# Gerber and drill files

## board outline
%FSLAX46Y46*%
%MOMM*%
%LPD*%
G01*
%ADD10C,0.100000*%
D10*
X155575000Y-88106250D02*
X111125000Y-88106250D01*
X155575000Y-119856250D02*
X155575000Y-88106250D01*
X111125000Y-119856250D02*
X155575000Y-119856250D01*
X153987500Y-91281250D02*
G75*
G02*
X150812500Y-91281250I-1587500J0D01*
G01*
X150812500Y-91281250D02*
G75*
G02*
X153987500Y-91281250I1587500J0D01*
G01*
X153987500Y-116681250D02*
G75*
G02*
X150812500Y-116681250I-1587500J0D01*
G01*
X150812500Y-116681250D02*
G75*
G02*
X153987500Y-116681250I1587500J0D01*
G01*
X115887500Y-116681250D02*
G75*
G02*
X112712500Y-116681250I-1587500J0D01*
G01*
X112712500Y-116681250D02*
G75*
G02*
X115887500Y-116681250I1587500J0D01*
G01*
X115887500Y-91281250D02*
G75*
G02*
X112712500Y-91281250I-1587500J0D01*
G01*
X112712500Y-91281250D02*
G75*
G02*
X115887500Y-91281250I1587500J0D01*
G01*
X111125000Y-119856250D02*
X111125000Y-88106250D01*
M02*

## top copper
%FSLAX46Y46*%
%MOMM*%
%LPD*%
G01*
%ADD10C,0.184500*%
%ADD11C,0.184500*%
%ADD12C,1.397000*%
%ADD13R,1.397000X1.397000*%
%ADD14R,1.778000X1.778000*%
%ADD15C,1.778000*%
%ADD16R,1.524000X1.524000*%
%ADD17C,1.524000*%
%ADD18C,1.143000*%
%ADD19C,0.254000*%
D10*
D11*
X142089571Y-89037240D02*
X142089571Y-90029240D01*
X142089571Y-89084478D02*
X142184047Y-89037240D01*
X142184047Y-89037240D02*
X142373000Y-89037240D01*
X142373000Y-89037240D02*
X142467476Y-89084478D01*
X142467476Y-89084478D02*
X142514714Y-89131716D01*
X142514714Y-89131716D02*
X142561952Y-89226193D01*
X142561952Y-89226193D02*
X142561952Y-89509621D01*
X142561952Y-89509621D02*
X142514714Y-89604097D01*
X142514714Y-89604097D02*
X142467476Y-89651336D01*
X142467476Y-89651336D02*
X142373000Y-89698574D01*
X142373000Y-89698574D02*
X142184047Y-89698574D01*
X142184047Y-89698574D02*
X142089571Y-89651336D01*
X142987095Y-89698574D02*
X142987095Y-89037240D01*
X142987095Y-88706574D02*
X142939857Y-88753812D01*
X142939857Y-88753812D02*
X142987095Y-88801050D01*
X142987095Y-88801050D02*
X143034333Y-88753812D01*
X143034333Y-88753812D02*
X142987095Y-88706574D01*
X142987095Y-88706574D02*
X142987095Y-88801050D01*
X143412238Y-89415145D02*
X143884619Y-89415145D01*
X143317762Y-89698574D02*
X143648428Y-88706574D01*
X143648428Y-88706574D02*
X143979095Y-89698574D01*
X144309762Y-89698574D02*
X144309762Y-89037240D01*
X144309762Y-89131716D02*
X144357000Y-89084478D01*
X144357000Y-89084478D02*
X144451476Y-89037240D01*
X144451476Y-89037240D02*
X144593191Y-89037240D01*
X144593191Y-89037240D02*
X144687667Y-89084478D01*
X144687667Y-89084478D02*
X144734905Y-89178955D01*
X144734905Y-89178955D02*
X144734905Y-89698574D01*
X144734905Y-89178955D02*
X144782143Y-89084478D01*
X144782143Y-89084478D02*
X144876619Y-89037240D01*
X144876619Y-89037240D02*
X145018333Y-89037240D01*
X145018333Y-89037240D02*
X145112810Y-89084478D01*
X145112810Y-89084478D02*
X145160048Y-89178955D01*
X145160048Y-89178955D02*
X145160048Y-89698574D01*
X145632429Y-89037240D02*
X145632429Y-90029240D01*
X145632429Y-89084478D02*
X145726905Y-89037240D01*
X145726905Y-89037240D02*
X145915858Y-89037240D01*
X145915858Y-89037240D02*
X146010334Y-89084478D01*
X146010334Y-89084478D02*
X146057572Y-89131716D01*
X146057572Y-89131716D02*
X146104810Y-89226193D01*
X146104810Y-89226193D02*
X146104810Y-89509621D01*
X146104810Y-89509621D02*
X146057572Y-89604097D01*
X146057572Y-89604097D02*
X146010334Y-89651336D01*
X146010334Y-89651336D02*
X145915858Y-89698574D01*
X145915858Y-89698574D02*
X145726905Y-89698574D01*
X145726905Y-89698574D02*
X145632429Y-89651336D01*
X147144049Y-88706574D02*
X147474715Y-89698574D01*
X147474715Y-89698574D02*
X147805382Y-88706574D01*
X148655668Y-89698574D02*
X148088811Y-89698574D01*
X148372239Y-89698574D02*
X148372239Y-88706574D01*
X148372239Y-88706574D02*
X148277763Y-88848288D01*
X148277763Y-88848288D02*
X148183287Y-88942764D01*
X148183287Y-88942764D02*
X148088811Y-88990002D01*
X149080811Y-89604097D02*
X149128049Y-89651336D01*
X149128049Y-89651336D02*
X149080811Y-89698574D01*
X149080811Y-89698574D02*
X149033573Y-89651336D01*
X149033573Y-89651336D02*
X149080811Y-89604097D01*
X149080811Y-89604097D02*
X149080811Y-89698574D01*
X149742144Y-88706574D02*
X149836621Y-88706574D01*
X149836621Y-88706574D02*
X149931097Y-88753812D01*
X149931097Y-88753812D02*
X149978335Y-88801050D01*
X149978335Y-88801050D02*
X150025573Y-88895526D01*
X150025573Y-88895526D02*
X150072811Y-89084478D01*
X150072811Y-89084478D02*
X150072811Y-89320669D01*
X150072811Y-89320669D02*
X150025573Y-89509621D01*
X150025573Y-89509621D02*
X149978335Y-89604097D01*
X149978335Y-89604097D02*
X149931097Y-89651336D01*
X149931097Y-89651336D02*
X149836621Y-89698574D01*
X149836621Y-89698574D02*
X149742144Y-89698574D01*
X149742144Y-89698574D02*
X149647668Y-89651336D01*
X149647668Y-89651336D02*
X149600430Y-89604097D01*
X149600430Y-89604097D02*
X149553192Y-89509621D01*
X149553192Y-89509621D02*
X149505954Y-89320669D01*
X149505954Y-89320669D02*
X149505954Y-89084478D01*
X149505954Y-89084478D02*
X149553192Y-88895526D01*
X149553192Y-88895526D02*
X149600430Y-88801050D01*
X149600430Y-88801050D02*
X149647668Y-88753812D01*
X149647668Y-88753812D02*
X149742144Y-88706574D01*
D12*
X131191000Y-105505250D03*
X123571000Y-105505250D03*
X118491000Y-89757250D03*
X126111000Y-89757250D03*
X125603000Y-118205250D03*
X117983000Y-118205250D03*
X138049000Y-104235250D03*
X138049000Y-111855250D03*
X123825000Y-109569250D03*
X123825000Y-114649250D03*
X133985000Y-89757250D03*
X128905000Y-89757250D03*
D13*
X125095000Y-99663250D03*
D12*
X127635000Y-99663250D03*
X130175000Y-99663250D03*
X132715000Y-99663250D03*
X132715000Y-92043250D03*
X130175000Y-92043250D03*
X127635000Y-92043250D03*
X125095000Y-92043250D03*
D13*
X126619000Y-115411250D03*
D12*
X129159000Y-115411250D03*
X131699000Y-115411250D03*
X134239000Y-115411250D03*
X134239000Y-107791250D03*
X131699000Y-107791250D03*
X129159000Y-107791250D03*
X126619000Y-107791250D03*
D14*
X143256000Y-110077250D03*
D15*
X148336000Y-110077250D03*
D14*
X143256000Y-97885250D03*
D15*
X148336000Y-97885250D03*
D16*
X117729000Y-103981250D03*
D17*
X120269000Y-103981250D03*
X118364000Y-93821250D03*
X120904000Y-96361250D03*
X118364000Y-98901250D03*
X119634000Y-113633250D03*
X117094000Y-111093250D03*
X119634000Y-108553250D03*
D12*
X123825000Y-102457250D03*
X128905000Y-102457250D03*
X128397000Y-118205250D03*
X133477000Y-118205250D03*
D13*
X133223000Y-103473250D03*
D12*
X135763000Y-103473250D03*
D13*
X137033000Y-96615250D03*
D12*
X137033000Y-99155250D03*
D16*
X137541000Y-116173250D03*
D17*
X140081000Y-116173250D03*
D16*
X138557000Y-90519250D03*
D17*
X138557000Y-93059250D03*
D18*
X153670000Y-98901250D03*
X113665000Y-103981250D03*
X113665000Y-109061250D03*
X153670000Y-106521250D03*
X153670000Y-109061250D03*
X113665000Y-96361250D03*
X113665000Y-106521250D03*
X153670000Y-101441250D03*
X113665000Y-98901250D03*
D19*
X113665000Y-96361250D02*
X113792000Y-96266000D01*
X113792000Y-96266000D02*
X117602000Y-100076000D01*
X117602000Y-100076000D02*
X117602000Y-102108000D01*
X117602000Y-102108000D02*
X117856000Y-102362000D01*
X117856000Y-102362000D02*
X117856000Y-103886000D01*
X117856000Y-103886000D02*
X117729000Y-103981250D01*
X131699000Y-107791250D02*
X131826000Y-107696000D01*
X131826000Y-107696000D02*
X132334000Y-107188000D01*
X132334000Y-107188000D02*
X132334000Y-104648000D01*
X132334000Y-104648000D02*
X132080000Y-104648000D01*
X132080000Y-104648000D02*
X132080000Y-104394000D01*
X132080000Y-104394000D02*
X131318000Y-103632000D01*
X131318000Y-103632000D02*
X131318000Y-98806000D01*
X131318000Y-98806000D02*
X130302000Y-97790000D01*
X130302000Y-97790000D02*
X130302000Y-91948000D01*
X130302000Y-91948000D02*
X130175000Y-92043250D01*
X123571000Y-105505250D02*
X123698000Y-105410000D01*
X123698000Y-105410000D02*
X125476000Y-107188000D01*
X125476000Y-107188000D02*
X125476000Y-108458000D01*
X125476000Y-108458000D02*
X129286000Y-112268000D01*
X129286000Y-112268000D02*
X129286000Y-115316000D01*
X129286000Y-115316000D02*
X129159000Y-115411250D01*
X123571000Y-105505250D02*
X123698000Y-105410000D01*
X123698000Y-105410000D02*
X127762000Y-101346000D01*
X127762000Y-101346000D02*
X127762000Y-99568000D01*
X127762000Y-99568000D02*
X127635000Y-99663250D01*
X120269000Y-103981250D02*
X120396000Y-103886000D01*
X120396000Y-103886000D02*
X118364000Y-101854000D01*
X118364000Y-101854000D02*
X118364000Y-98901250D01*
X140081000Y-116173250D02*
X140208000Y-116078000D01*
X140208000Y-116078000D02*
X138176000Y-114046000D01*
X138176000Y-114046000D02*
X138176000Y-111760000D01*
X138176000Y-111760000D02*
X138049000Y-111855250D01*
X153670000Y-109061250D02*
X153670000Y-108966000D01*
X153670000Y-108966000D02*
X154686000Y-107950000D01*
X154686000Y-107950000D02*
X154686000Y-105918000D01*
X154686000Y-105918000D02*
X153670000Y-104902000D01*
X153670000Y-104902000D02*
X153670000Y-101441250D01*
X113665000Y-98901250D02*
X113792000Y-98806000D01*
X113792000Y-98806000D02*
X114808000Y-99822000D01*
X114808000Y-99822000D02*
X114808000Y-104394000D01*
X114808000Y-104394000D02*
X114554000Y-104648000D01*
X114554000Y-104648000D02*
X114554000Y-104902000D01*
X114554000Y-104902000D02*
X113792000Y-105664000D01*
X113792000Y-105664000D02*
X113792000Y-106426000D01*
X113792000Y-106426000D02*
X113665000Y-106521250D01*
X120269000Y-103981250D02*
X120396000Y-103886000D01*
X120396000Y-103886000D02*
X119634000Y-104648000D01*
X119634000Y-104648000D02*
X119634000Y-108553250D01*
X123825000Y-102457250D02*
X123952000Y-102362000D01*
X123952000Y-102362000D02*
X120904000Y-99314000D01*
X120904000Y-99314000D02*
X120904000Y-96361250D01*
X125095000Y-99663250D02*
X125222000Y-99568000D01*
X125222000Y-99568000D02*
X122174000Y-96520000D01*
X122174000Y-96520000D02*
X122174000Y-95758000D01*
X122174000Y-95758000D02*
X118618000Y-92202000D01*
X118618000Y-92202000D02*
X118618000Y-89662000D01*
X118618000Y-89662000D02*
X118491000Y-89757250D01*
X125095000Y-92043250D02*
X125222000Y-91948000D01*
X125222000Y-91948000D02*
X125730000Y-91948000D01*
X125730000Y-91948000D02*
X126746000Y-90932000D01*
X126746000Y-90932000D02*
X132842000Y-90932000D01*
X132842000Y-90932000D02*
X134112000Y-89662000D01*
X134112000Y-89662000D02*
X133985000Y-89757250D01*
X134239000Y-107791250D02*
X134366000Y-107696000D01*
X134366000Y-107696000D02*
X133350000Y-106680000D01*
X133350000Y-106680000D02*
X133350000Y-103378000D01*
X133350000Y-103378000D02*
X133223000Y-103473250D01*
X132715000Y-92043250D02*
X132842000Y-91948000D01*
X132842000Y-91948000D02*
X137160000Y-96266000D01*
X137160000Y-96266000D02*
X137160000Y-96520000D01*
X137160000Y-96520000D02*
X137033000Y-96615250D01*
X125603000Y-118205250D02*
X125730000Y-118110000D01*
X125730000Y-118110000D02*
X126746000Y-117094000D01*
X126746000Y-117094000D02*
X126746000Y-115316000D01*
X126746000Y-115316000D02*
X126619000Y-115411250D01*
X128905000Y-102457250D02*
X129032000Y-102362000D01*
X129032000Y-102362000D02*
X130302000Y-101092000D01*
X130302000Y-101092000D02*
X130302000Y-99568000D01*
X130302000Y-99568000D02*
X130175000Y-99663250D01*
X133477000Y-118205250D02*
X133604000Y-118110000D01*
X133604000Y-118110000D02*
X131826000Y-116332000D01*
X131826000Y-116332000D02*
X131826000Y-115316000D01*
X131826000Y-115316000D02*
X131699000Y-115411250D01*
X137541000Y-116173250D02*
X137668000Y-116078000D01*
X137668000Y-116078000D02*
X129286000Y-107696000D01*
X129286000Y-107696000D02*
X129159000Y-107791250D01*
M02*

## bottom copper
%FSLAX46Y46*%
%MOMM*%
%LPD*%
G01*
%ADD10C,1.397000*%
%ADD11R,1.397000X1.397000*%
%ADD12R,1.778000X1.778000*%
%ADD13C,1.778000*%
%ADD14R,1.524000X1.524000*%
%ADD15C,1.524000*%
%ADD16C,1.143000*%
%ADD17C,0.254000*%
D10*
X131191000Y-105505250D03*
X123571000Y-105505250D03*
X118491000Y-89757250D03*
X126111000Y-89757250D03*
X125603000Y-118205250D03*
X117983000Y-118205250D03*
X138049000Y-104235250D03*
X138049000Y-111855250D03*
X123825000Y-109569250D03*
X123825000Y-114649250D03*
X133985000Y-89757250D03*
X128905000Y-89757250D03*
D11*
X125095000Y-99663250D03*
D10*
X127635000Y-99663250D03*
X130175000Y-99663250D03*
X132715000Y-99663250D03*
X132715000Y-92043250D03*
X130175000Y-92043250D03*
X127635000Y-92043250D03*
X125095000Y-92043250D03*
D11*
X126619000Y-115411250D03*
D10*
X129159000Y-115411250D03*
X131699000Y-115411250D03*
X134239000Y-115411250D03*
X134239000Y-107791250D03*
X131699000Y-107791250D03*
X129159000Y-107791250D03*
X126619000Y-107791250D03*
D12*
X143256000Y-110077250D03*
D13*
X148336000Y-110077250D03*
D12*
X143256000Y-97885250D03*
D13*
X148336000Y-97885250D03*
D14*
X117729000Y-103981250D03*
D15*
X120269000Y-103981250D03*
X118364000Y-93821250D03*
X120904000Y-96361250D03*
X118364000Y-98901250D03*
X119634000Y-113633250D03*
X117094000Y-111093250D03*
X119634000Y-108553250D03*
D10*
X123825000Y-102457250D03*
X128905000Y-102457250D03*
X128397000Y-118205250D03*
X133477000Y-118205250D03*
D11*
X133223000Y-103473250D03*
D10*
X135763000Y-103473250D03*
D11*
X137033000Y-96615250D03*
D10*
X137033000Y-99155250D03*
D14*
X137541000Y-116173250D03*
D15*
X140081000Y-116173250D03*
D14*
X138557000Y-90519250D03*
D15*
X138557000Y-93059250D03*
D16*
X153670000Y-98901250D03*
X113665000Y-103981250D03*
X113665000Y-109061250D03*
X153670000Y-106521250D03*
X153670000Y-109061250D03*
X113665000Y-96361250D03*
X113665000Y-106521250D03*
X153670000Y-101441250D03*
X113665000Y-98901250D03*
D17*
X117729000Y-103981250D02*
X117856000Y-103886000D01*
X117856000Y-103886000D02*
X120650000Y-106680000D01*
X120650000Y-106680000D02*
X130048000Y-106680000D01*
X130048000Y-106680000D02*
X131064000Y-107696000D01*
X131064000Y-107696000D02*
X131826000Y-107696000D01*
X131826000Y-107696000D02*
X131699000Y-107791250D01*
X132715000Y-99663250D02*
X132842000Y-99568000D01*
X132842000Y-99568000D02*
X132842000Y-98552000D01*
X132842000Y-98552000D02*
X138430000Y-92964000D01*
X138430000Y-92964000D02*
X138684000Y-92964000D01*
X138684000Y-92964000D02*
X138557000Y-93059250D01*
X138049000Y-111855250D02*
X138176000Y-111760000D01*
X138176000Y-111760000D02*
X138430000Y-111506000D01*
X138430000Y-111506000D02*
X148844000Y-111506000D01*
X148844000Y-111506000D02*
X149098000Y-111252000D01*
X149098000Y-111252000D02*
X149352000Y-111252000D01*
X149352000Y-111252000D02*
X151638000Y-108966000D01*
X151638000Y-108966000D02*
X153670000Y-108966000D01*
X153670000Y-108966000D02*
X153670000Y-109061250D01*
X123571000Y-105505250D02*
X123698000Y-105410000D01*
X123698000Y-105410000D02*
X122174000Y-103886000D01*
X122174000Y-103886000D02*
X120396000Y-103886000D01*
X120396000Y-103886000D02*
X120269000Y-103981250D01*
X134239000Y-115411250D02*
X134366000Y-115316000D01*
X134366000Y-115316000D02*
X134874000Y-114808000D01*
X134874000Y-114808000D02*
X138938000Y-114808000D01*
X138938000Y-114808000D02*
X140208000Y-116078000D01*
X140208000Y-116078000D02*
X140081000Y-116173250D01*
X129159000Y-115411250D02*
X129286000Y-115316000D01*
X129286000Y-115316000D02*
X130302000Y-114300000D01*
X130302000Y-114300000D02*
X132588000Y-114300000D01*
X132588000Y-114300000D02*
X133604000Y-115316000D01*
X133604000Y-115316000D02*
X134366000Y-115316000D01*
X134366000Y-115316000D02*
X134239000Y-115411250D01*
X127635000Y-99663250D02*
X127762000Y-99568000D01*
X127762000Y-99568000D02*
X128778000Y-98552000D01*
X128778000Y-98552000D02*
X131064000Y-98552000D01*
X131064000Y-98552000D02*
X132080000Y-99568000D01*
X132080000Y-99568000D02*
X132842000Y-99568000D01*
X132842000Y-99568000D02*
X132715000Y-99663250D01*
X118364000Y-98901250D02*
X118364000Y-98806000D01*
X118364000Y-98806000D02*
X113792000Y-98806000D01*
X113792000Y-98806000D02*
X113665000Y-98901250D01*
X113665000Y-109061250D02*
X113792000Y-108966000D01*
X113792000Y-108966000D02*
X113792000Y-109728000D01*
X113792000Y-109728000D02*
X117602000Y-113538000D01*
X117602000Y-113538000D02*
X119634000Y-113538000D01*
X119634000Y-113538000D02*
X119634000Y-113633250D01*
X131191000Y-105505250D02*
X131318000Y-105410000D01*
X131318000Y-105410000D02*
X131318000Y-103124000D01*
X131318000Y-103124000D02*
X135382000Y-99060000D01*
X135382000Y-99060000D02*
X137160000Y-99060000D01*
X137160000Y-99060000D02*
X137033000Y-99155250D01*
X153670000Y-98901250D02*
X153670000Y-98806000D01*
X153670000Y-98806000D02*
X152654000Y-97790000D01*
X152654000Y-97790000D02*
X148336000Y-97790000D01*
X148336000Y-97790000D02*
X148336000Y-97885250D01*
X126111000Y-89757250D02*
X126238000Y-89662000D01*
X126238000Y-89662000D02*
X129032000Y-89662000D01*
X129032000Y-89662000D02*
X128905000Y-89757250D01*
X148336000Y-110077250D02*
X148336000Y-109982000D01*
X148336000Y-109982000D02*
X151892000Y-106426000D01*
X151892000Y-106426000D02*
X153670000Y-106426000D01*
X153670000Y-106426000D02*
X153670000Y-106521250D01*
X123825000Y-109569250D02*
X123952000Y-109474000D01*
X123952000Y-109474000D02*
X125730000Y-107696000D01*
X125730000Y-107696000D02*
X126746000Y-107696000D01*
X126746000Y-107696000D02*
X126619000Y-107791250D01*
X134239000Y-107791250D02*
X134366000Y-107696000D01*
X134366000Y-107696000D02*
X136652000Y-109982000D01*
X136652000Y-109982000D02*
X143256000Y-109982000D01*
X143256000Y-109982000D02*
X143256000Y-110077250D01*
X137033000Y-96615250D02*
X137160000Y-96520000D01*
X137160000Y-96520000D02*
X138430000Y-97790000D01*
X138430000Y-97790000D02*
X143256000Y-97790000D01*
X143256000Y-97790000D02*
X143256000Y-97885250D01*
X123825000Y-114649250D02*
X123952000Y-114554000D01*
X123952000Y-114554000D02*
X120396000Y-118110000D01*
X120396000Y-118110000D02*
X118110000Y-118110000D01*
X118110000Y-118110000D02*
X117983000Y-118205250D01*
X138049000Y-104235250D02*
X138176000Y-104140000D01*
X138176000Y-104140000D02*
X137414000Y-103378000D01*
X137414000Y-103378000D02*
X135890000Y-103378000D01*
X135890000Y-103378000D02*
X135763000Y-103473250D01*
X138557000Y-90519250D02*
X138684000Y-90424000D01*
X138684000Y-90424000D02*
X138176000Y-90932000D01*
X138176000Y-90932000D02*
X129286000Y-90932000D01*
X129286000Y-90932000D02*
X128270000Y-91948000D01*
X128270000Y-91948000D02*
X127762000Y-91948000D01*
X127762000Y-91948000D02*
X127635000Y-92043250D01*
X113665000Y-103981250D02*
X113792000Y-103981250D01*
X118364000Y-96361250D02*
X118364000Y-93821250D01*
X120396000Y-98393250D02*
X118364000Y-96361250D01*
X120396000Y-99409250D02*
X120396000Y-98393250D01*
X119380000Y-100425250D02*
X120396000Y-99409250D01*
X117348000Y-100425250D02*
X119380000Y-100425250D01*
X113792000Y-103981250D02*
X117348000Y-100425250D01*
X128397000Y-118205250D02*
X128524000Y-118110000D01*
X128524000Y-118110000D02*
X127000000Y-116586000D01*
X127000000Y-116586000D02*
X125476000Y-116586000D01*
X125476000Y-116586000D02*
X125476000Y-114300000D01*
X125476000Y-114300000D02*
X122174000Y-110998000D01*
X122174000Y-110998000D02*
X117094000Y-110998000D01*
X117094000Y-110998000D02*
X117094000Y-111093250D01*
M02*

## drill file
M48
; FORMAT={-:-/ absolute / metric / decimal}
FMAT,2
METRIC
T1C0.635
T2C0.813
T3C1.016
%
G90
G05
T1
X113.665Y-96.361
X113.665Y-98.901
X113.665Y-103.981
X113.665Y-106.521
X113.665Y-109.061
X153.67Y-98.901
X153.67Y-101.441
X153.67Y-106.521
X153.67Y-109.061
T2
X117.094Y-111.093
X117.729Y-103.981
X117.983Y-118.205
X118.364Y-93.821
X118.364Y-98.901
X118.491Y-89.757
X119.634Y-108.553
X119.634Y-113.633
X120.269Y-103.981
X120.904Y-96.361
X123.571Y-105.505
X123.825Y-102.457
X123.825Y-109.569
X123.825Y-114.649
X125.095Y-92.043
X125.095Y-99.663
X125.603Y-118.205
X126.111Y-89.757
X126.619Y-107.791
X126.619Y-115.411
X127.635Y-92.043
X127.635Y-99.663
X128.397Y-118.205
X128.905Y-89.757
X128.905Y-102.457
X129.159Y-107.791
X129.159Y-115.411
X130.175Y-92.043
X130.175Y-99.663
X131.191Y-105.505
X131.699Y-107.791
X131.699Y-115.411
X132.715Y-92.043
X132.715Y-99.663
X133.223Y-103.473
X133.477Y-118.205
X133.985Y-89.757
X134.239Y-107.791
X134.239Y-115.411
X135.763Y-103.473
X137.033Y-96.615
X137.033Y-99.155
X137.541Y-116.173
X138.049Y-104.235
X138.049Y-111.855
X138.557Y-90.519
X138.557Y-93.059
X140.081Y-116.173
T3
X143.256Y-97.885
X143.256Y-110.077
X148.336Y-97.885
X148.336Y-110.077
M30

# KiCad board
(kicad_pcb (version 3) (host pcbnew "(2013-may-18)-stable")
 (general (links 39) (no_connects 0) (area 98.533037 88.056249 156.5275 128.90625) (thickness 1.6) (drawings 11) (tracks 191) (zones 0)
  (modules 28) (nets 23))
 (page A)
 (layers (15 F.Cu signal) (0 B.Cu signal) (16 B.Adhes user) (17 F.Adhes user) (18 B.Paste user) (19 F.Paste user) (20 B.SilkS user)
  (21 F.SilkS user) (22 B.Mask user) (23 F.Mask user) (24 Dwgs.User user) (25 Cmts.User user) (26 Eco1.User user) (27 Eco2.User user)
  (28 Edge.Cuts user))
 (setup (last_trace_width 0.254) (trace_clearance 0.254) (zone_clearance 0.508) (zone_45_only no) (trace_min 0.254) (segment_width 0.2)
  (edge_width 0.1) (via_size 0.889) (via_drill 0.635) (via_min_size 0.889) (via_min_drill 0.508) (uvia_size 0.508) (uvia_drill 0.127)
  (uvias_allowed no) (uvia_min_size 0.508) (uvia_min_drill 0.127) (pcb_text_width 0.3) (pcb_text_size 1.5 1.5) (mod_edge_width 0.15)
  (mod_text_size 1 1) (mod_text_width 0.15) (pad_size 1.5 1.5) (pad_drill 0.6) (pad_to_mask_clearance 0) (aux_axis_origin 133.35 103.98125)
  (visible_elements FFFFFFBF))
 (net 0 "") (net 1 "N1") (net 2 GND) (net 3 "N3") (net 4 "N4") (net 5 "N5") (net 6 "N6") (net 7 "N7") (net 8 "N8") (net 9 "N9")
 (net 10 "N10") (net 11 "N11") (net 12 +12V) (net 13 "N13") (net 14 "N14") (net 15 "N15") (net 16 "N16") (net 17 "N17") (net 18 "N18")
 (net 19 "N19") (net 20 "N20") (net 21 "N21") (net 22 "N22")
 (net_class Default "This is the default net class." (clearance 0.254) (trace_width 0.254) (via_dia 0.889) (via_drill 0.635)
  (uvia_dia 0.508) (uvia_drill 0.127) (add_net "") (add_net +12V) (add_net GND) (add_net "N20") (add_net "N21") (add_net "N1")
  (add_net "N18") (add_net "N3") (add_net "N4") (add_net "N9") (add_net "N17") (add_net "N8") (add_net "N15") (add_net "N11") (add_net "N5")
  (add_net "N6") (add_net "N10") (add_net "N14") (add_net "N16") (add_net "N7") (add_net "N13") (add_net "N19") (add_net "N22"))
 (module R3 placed (layer F.Cu) (at 127.381 105.50525 180) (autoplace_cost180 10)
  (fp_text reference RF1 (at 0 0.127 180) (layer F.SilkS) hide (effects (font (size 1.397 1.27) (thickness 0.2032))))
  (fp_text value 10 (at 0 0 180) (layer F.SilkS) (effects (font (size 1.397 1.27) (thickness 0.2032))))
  (pad 1 thru_hole circle (at -3.81 0 180) (size 1.397 1.397) (drill 0.8128) (layers *.Cu *.Mask F.SilkS) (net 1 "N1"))
  (pad 2 thru_hole circle (at 3.81 0 180) (size 1.397 1.397) (drill 0.8128) (layers *.Cu *.Mask F.SilkS) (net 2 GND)))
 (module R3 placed (layer F.Cu) (at 122.301 89.75725) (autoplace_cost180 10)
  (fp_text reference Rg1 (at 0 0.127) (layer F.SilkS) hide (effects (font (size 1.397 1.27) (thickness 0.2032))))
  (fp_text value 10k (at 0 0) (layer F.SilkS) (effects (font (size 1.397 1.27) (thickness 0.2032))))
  (pad 1 thru_hole circle (at -3.81 0) (size 1.397 1.397) (drill 0.8128) (layers *.Cu *.Mask F.SilkS) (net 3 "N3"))
  (pad 2 thru_hole circle (at 3.81 0) (size 1.397 1.397) (drill 0.8128) (layers *.Cu *.Mask F.SilkS) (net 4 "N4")))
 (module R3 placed (layer F.Cu) (at 121.793 118.20525 180) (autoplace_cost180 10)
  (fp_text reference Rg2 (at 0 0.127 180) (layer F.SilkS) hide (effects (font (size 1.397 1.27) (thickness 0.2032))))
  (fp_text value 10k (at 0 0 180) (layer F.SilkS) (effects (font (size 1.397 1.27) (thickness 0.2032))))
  (pad 1 thru_hole circle (at -3.81 0 180) (size 1.397 1.397) (drill 0.8128) (layers *.Cu *.Mask F.SilkS) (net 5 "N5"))
  (pad 2 thru_hole circle (at 3.81 0 180) (size 1.397 1.397) (drill 0.8128) (layers *.Cu *.Mask F.SilkS) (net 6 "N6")))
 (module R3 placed (layer F.Cu) (at 138.049 108.04525 270) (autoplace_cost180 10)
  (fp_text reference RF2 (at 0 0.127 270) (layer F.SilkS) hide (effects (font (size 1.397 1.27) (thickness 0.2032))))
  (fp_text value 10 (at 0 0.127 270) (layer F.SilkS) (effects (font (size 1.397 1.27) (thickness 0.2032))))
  (pad 1 thru_hole circle (at -3.81 0 270) (size 1.397 1.397) (drill 0.8128) (layers *.Cu *.Mask F.SilkS) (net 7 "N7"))
  (pad 2 thru_hole circle (at 3.81 0 270) (size 1.397 1.397) (drill 0.8128) (layers *.Cu *.Mask F.SilkS) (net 2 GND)))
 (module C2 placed (layer F.Cu) (at 123.825 112.10925 270)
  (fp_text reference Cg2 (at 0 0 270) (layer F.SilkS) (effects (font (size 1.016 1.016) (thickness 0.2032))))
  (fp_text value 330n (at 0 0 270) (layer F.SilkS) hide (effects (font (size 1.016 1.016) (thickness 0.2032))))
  (pad 1 thru_hole circle (at -2.54 0 270) (size 1.397 1.397) (drill 0.8128) (layers *.Cu *.Mask F.SilkS) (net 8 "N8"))
  (pad 2 thru_hole circle (at 2.54 0 270) (size 1.397 1.397) (drill 0.8128) (layers *.Cu *.Mask F.SilkS) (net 6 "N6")))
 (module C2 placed (layer F.Cu) (at 131.445 89.75725 180)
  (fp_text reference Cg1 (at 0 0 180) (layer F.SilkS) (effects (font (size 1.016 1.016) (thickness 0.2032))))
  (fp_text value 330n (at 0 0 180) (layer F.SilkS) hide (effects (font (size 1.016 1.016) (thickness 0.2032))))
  (pad 1 thru_hole circle (at -2.54 0 180) (size 1.397 1.397) (drill 0.8128) (layers *.Cu *.Mask F.SilkS) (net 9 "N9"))
  (pad 2 thru_hole circle (at 2.54 0 180) (size 1.397 1.397) (drill 0.8128) (layers *.Cu *.Mask F.SilkS) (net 4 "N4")))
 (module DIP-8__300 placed (layer F.Cu) (at 128.905 95.85325)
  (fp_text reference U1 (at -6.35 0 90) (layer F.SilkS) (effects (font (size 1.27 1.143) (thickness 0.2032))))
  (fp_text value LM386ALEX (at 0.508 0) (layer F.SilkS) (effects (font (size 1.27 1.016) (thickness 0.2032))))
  (pad 1 thru_hole rect (at -3.81 3.81) (size 1.397 1.397) (drill 0.8128) (layers *.Cu *.Mask F.SilkS) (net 3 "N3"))
  (pad 2 thru_hole circle (at -1.27 3.81) (size 1.397 1.397) (drill 0.8128) (layers *.Cu *.Mask F.SilkS) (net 2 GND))
  (pad 3 thru_hole circle (at 1.27 3.81) (size 1.397 1.397) (drill 0.8128) (layers *.Cu *.Mask F.SilkS) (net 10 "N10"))
  (pad 4 thru_hole circle (at 3.81 3.81) (size 1.397 1.397) (drill 0.8128) (layers *.Cu *.Mask F.SilkS) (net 2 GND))
  (pad 5 thru_hole circle (at 3.81 -3.81) (size 1.397 1.397) (drill 0.8128) (layers *.Cu *.Mask F.SilkS) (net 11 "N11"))
  (pad 6 thru_hole circle (at 1.27 -3.81) (size 1.397 1.397) (drill 0.8128) (layers *.Cu *.Mask F.SilkS) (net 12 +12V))
  (pad 7 thru_hole circle (at -1.27 -3.81) (size 1.397 1.397) (drill 0.8128) (layers *.Cu *.Mask F.SilkS) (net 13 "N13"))
  (pad 8 thru_hole circle (at -3.81 -3.81) (size 1.397 1.397) (drill 0.8128) (layers *.Cu *.Mask F.SilkS) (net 9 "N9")))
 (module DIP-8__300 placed (layer F.Cu) (at 130.429 111.60125)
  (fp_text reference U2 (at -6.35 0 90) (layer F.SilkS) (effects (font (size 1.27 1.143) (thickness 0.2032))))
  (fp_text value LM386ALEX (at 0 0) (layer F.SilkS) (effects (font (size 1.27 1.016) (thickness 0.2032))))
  (pad 1 thru_hole rect (at -3.81 3.81) (size 1.397 1.397) (drill 0.8128) (layers *.Cu *.Mask F.SilkS) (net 5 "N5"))
  (pad 2 thru_hole circle (at -1.27 3.81) (size 1.397 1.397) (drill 0.8128) (layers *.Cu *.Mask F.SilkS) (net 2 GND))
  (pad 3 thru_hole circle (at 1.27 3.81) (size 1.397 1.397) (drill 0.8128) (layers *.Cu *.Mask F.SilkS) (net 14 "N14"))
  (pad 4 thru_hole circle (at 3.81 3.81) (size 1.397 1.397) (drill 0.8128) (layers *.Cu *.Mask F.SilkS) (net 2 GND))
  (pad 5 thru_hole circle (at 3.81 -3.81) (size 1.397 1.397) (drill 0.8128) (layers *.Cu *.Mask F.SilkS) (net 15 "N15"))
  (pad 6 thru_hole circle (at 1.27 -3.81) (size 1.397 1.397) (drill 0.8128) (layers *.Cu *.Mask F.SilkS) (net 12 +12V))
  (pad 7 thru_hole circle (at -1.27 -3.81) (size 1.397 1.397) (drill 0.8128) (layers *.Cu *.Mask F.SilkS) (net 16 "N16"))
  (pad 8 thru_hole circle (at -3.81 -3.81) (size 1.397 1.397) (drill 0.8128) (layers *.Cu *.Mask F.SilkS) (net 8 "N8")))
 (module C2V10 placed (layer F.Cu) (at 145.796 110.07725)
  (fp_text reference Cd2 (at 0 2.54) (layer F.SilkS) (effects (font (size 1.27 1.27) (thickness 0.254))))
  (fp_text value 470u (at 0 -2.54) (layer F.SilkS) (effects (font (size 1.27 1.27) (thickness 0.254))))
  (pad 1 thru_hole rect (at -2.54 0) (size 1.778 1.778) (drill 1.016) (layers *.Cu *.Mask F.SilkS) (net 15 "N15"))
  (pad 2 thru_hole circle (at 2.54 0) (size 1.778 1.778) (drill 1.016) (layers *.Cu *.Mask F.SilkS) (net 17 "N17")))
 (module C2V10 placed (layer F.Cu) (at 145.796 97.88525)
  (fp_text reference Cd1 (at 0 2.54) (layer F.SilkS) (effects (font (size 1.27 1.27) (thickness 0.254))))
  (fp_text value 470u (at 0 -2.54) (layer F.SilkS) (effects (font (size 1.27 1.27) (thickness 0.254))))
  (pad 1 thru_hole rect (at -2.54 0) (size 1.778 1.778) (drill 1.016) (layers *.Cu *.Mask F.SilkS) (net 11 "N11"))
  (pad 2 thru_hole circle (at 2.54 0) (size 1.778 1.778) (drill 1.016) (layers *.Cu *.Mask F.SilkS) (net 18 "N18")))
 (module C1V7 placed (layer F.Cu) (at 118.999 103.98125)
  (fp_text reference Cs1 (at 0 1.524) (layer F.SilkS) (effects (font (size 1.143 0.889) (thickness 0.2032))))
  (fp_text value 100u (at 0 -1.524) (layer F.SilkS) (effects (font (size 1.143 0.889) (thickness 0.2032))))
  (pad 1 thru_hole rect (at -1.27 0) (size 1.524 1.524) (drill 0.8128) (layers *.Cu *.Mask F.SilkS) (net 12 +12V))
  (pad 2 thru_hole circle (at 1.27 0) (size 1.524 1.524) (drill 0.8128) (layers *.Cu *.Mask F.SilkS) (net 2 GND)))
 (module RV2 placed (layer F.Cu) (at 119.634 96.36125 270) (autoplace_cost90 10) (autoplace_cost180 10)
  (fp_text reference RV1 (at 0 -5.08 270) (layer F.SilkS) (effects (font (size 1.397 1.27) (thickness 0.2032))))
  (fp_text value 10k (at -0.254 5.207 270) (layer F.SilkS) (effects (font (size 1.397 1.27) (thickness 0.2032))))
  (pad 1 thru_hole circle (at -2.54 1.27 270) (size 1.524 1.524) (drill 0.8128) (layers *.Cu *.Mask F.SilkS) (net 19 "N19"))
  (pad 2 thru_hole circle (at 0 -1.27 270) (size 1.524 1.524) (drill 0.8128) (layers *.Cu *.Mask F.SilkS) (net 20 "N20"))
  (pad 3 thru_hole circle (at 2.54 1.27 270) (size 1.524 1.524) (drill 0.8128) (layers *.Cu *.Mask F.SilkS) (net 2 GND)))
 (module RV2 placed (layer F.Cu) (at 118.364 111.09325 90) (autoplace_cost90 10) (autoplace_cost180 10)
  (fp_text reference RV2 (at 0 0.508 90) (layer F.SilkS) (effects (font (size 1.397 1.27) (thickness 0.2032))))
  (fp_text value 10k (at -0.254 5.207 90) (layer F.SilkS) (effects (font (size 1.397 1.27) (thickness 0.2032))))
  (pad 1 thru_hole circle (at -2.54 1.27 90) (size 1.524 1.524) (drill 0.8128) (layers *.Cu *.Mask F.SilkS) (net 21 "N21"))
  (pad 2 thru_hole circle (at 0 -1.27 90) (size 1.524 1.524) (drill 0.8128) (layers *.Cu *.Mask F.SilkS) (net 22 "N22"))
  (pad 3 thru_hole circle (at 2.54 1.27 90) (size 1.524 1.524) (drill 0.8128) (layers *.Cu *.Mask F.SilkS) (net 2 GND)))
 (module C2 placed (layer F.Cu) (at 126.365 102.45725)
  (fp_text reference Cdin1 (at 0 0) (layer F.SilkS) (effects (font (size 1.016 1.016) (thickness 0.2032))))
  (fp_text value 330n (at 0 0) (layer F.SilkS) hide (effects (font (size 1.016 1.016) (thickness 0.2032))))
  (pad 1 thru_hole circle (at -2.54 0) (size 1.397 1.397) (drill 0.8128) (layers *.Cu *.Mask F.SilkS) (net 20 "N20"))
  (pad 2 thru_hole circle (at 2.54 0) (size 1.397 1.397) (drill 0.8128) (layers *.Cu *.Mask F.SilkS) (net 10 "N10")))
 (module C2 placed (layer F.Cu) (at 130.937 118.20525)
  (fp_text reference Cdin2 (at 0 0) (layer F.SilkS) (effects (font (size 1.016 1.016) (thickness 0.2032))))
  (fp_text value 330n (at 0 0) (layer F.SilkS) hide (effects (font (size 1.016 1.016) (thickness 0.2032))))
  (pad 1 thru_hole circle (at -2.54 0) (size 1.397 1.397) (drill 0.8128) (layers *.Cu *.Mask F.SilkS) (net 22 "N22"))
  (pad 2 thru_hole circle (at 2.54 0) (size 1.397 1.397) (drill 0.8128) (layers *.Cu *.Mask F.SilkS) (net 14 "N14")))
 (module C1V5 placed (layer F.Cu) (at 134.493 103.47325)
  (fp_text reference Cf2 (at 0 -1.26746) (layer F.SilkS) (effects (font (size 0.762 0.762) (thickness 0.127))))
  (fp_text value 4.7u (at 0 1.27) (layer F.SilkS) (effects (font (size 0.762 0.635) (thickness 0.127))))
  (pad 1 thru_hole rect (at -1.27 0) (size 1.397 1.397) (drill 0.8128) (layers *.Cu *.Mask F.SilkS) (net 15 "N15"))
  (pad 2 thru_hole circle (at 1.27 0) (size 1.397 1.397) (drill 0.8128) (layers *.Cu *.Mask F.SilkS) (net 7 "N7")))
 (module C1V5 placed (layer F.Cu) (at 137.033 97.88525 270)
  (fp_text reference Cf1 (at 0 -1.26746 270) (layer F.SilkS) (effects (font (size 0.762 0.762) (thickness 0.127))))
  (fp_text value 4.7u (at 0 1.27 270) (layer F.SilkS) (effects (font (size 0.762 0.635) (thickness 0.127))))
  (pad 1 thru_hole rect (at -1.27 0 270) (size 1.397 1.397) (drill 0.8128) (layers *.Cu *.Mask F.SilkS) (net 11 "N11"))
  (pad 2 thru_hole circle (at 1.27 0 270) (size 1.397 1.397) (drill 0.8128) (layers *.Cu *.Mask F.SilkS) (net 1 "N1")))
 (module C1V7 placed (layer F.Cu) (at 138.811 116.17325)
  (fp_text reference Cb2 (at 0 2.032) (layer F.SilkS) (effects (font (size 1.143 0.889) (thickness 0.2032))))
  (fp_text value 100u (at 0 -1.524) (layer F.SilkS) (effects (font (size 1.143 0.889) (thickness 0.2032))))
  (pad 1 thru_hole rect (at -1.27 0) (size 1.524 1.524) (drill 0.8128) (layers *.Cu *.Mask F.SilkS) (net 16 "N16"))
  (pad 2 thru_hole circle (at 1.27 0) (size 1.524 1.524) (drill 0.8128) (layers *.Cu *.Mask F.SilkS) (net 2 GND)))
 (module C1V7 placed (layer F.Cu) (at 138.557 91.78925 270)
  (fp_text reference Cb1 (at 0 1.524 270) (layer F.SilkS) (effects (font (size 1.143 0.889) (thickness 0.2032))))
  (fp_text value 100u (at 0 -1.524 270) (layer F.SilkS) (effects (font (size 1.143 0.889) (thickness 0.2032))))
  (pad 1 thru_hole rect (at -1.27 0 270) (size 1.524 1.524) (drill 0.8128) (layers *.Cu *.Mask F.SilkS) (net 13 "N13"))
  (pad 2 thru_hole circle (at 1.27 0 270) (size 1.524 1.524) (drill 0.8128) (layers *.Cu *.Mask F.SilkS) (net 2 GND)))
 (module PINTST (layer F.Cu) (at 153.67 98.90125)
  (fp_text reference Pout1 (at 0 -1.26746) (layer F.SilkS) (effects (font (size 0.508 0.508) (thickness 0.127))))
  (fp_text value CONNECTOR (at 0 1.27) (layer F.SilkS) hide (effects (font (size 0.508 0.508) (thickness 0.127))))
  (pad 1 thru_hole circle (at 0 0) (size 1.143 1.143) (drill 0.635) (layers *.Cu *.Mask F.SilkS) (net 18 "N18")))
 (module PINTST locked (layer F.Cu) (at 113.665 103.98125)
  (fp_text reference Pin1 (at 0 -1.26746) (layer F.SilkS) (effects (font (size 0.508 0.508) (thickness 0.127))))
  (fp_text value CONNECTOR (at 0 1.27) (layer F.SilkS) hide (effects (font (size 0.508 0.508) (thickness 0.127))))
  (pad 1 thru_hole circle (at 0 0) (size 1.143 1.143) (drill 0.635) (layers *.Cu *.Mask F.SilkS) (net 19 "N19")))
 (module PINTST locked (layer F.Cu) (at 113.665 109.06125)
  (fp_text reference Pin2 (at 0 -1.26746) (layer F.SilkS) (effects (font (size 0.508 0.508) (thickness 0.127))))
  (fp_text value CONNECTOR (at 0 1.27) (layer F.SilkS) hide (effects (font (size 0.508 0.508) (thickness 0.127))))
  (pad 1 thru_hole circle (at 0 0) (size 1.143 1.143) (drill 0.635) (layers *.Cu *.Mask F.SilkS) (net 21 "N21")))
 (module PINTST (layer F.Cu) (at 153.67 106.52125)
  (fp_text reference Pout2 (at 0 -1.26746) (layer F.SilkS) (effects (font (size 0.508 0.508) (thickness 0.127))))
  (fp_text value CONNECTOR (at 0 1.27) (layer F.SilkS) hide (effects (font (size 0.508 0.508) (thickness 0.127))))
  (pad 1 thru_hole circle (at 0 0) (size 1.143 1.143) (drill 0.635) (layers *.Cu *.Mask F.SilkS) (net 17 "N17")))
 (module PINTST (layer F.Cu) (at 153.67 109.06125)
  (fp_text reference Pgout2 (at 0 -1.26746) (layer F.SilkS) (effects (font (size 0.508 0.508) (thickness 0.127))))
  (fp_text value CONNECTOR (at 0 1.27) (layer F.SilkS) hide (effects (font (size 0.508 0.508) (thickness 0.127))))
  (pad 1 thru_hole circle (at 0 0) (size 1.143 1.143) (drill 0.635) (layers *.Cu *.Mask F.SilkS) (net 2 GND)))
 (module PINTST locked (layer F.Cu) (at 113.665 96.36125)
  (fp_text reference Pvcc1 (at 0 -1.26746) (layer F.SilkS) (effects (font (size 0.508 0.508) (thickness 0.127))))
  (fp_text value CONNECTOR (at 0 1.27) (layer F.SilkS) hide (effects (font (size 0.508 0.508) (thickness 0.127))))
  (pad 1 thru_hole circle (at 0 0) (size 1.143 1.143) (drill 0.635) (layers *.Cu *.Mask F.SilkS) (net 12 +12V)))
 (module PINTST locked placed (layer F.Cu) (at 113.665 106.52125)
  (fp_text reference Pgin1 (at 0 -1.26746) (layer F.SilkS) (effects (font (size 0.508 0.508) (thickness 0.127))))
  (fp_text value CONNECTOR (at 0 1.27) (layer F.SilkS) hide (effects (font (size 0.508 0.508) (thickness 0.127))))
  (pad 1 thru_hole circle (at 0 0) (size 1.143 1.143) (drill 0.635) (layers *.Cu *.Mask F.SilkS) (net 2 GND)))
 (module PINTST (layer F.Cu) (at 153.67 101.44125)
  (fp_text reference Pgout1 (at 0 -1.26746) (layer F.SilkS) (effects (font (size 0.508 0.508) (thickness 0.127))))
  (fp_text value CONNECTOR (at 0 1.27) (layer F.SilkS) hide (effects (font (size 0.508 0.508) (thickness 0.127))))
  (pad 1 thru_hole circle (at 0 0) (size 1.143 1.143) (drill 0.635) (layers *.Cu *.Mask F.SilkS) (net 2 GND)))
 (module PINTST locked (layer F.Cu) (at 113.665 98.90125)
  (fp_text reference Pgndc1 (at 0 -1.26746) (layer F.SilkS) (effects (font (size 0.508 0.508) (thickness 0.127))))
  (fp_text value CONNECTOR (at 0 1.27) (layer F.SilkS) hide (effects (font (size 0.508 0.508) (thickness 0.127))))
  (pad 1 thru_hole circle (at 0 0) (size 1.143 1.143) (drill 0.635) (layers *.Cu *.Mask F.SilkS) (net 2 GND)))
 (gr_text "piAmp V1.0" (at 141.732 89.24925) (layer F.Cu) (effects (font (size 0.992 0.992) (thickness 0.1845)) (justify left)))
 (gr_line (start 155.575 88.10625) (end 111.125 88.10625) (angle 90) (layer Edge.Cuts) (width 0.1))
 (gr_line (start 155.575 119.85625) (end 155.575 88.10625) (angle 90) (layer Edge.Cuts) (width 0.1))
 (gr_line (start 111.125 119.85625) (end 155.575 119.85625) (angle 90) (layer Edge.Cuts) (width 0.1))
 (gr_circle (center 152.4 91.28125) (end 153.9875 91.28125) (layer Edge.Cuts) (width 0.1))
 (gr_circle (center 152.4 116.68125) (end 153.9875 116.68125) (layer Edge.Cuts) (width 0.1))
 (gr_circle (center 114.3 116.68125) (end 112.7125 116.68125) (layer Edge.Cuts) (width 0.1))
 (gr_circle (center 114.3 91.28125) (end 112.7125 91.28125) (layer Edge.Cuts) (width 0.1))
 (gr_line (start 111.125 119.85625) (end 111.125 88.10625) (angle 90) (layer Edge.Cuts) (width 0.1))
 (segment (start 117.729 103.98125) (end 117.856 103.886) (width 0.254) (layer B.Cu) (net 12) (status 80000))
 (segment (start 117.856 103.886) (end 120.65 106.68) (width 0.254) (layer B.Cu) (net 12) (status 80000))
 (segment (start 120.65 106.68) (end 130.048 106.68) (width 0.254) (layer B.Cu) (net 12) (status 80000))
 (segment (start 130.048 106.68) (end 131.064 107.696) (width 0.254) (layer B.Cu) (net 12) (status 80000))
 (segment (start 131.064 107.696) (end 131.826 107.696) (width 0.254) (layer B.Cu) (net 12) (status 80000))
 (segment (start 131.826 107.696) (end 131.699 107.79125) (width 0.254) (layer B.Cu) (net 12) (status 80000))
 (segment (start 113.665 96.36125) (end 113.792 96.266) (width 0.254) (layer F.Cu) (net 12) (status 80000))
 (segment (start 113.792 96.266) (end 117.602 100.076) (width 0.254) (layer F.Cu) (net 12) (status 80000))
 (segment (start 117.602 100.076) (end 117.602 102.108) (width 0.254) (layer F.Cu) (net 12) (status 80000))
 (segment (start 117.602 102.108) (end 117.856 102.362) (width 0.254) (layer F.Cu) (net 12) (status 80000))
 (segment (start 117.856 102.362) (end 117.856 103.886) (width 0.254) (layer F.Cu) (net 12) (status 80000))
 (segment (start 117.856 103.886) (end 117.729 103.98125) (width 0.254) (layer F.Cu) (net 12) (status 80000))
 (segment (start 131.699 107.79125) (end 131.826 107.696) (width 0.254) (layer F.Cu) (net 12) (status 80000))
 (segment (start 131.826 107.696) (end 132.334 107.188) (width 0.254) (layer F.Cu) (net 12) (status 80000))
 (segment (start 132.334 107.188) (end 132.334 104.648) (width 0.254) (layer F.Cu) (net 12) (status 80000))
 (segment (start 132.334 104.648) (end 132.08 104.648) (width 0.254) (layer F.Cu) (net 12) (status 80000))
 (segment (start 132.08 104.648) (end 132.08 104.394) (width 0.254) (layer F.Cu) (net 12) (status 80000))
 (segment (start 132.08 104.394) (end 131.318 103.632) (width 0.254) (layer F.Cu) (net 12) (status 80000))
 (segment (start 131.318 103.632) (end 131.318 98.806) (width 0.254) (layer F.Cu) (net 12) (status 80000))
 (segment (start 131.318 98.806) (end 130.302 97.79) (width 0.254) (layer F.Cu) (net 12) (status 80000))
 (segment (start 130.302 97.79) (end 130.302 91.948) (width 0.254) (layer F.Cu) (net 12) (status 80000))
 (segment (start 130.302 91.948) (end 130.175 92.04325) (width 0.254) (layer F.Cu) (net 12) (status 80000))
 (segment (start 132.715 99.66325) (end 132.842 99.568) (width 0.254) (layer B.Cu) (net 2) (status 80000))
 (segment (start 132.842 99.568) (end 132.842 98.552) (width 0.254) (layer B.Cu) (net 2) (status 80000))
 (segment (start 132.842 98.552) (end 138.43 92.964) (width 0.254) (layer B.Cu) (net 2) (status 80000))
 (segment (start 138.43 92.964) (end 138.684 92.964) (width 0.254) (layer B.Cu) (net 2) (status 80000))
 (segment (start 138.684 92.964) (end 138.557 93.05925) (width 0.254) (layer B.Cu) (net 2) (status 80000))
 (segment (start 123.571 105.50525) (end 123.698 105.41) (width 0.254) (layer F.Cu) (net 2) (status 80000))
 (segment (start 123.698 105.41) (end 125.476 107.188) (width 0.254) (layer F.Cu) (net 2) (status 80000))
 (segment (start 125.476 107.188) (end 125.476 108.458) (width 0.254) (layer F.Cu) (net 2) (status 80000))
 (segment (start 125.476 108.458) (end 129.286 112.268) (width 0.254) (layer F.Cu) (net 2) (status 80000))
 (segment (start 129.286 112.268) (end 129.286 115.316) (width 0.254) (layer F.Cu) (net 2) (status 80000))
 (segment (start 129.286 115.316) (end 129.159 115.41125) (width 0.254) (layer F.Cu) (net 2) (status 80000))
 (segment (start 138.049 111.85525) (end 138.176 111.76) (width 0.254) (layer B.Cu) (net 2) (status 80000))
 (segment (start 138.176 111.76) (end 138.43 111.506) (width 0.254) (layer B.Cu) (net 2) (status 80000))
 (segment (start 138.43 111.506) (end 148.844 111.506) (width 0.254) (layer B.Cu) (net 2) (status 80000))
 (segment (start 148.844 111.506) (end 149.098 111.252) (width 0.254) (layer B.Cu) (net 2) (status 80000))
 (segment (start 149.098 111.252) (end 149.352 111.252) (width 0.254) (layer B.Cu) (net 2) (status 80000))
 (segment (start 149.352 111.252) (end 151.638 108.966) (width 0.254) (layer B.Cu) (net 2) (status 80000))
 (segment (start 151.638 108.966) (end 153.67 108.966) (width 0.254) (layer B.Cu) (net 2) (status 80000))
 (segment (start 153.67 108.966) (end 153.67 109.06125) (width 0.254) (layer B.Cu) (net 2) (status 80000))
 (segment (start 123.571 105.50525) (end 123.698 105.41) (width 0.254) (layer F.Cu) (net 2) (status 80000))
 (segment (start 123.698 105.41) (end 127.762 101.346) (width 0.254) (layer F.Cu) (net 2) (status 80000))
 (segment (start 127.762 101.346) (end 127.762 99.568) (width 0.254) (layer F.Cu) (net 2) (status 80000))
 (segment (start 127.762 99.568) (end 127.635 99.66325) (width 0.254) (layer F.Cu) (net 2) (status 80000))
 (segment (start 120.269 103.98125) (end 120.396 103.886) (width 0.254) (layer F.Cu) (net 2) (status 80000))
 (segment (start 120.396 103.886) (end 118.364 101.854) (width 0.254) (layer F.Cu) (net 2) (status 80000))
 (segment (start 118.364 101.854) (end 118.364 98.90125) (width 0.254) (layer F.Cu) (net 2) (status 80000))
 (segment (start 140.081 116.17325) (end 140.208 116.078) (width 0.254) (layer F.Cu) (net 2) (status 80000))
 (segment (start 140.208 116.078) (end 138.176 114.046) (width 0.254) (layer F.Cu) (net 2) (status 80000))
 (segment (start 138.176 114.046) (end 138.176 111.76) (width 0.254) (layer F.Cu) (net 2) (status 80000))
 (segment (start 138.176 111.76) (end 138.049 111.85525) (width 0.254) (layer F.Cu) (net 2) (status 80000))
 (segment (start 123.571 105.50525) (end 123.698 105.41) (width 0.254) (layer B.Cu) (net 2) (status 80000))
 (segment (start 123.698 105.41) (end 122.174 103.886) (width 0.254) (layer B.Cu) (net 2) (status 80000))
 (segment (start 122.174 103.886) (end 120.396 103.886) (width 0.254) (layer B.Cu) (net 2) (status 80000))
 (segment (start 120.396 103.886) (end 120.269 103.98125) (width 0.254) (layer B.Cu) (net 2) (status 80000))
 (segment (start 134.239 115.41125) (end 134.366 115.316) (width 0.254) (layer B.Cu) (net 2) (status 80000))
 (segment (start 134.366 115.316) (end 134.874 114.808) (width 0.254) (layer B.Cu) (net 2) (status 80000))
 (segment (start 134.874 114.808) (end 138.938 114.808) (width 0.254) (layer B.Cu) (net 2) (status 80000))
 (segment (start 138.938 114.808) (end 140.208 116.078) (width 0.254) (layer B.Cu) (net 2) (status 80000))
 (segment (start 140.208 116.078) (end 140.081 116.17325) (width 0.254) (layer B.Cu) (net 2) (status 80000))
 (segment (start 153.67 109.06125) (end 153.67 108.966) (width 0.254) (layer F.Cu) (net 2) (status 80000))
 (segment (start 153.67 108.966) (end 154.686 107.95) (width 0.254) (layer F.Cu) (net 2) (status 80000))
 (segment (start 154.686 107.95) (end 154.686 105.918) (width 0.254) (layer F.Cu) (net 2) (status 80000))
 (segment (start 154.686 105.918) (end 153.67 104.902) (width 0.254) (layer F.Cu) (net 2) (status 80000))
 (segment (start 153.67 104.902) (end 153.67 101.44125) (width 0.254) (layer F.Cu) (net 2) (status 80000))
 (segment (start 113.665 98.90125) (end 113.792 98.806) (width 0.254) (layer F.Cu) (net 2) (status 80000))
 (segment (start 113.792 98.806) (end 114.808 99.822) (width 0.254) (layer F.Cu) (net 2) (status 80000))
 (segment (start 114.808 99.822) (end 114.808 104.394) (width 0.254) (layer F.Cu) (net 2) (status 80000))
 (segment (start 114.808 104.394) (end 114.554 104.648) (width 0.254) (layer F.Cu) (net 2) (status 80000))
 (segment (start 114.554 104.648) (end 114.554 104.902) (width 0.254) (layer F.Cu) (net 2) (status 80000))
 (segment (start 114.554 104.902) (end 113.792 105.664) (width 0.254) (layer F.Cu) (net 2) (status 80000))
 (segment (start 113.792 105.664) (end 113.792 106.426) (width 0.254) (layer F.Cu) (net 2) (status 80000))
 (segment (start 113.792 106.426) (end 113.665 106.52125) (width 0.254) (layer F.Cu) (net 2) (status 80000))
 (segment (start 120.269 103.98125) (end 120.396 103.886) (width 0.254) (layer F.Cu) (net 2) (status 80000))
 (segment (start 120.396 103.886) (end 119.634 104.648) (width 0.254) (layer F.Cu) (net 2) (status 80000))
 (segment (start 119.634 104.648) (end 119.634 108.55325) (width 0.254) (layer F.Cu) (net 2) (status 80000))
 (segment (start 129.159 115.41125) (end 129.286 115.316) (width 0.254) (layer B.Cu) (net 2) (status 80000))
 (segment (start 129.286 115.316) (end 130.302 114.3) (width 0.254) (layer B.Cu) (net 2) (status 80000))
 (segment (start 130.302 114.3) (end 132.588 114.3) (width 0.254) (layer B.Cu) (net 2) (status 80000))
 (segment (start 132.588 114.3) (end 133.604 115.316) (width 0.254) (layer B.Cu) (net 2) (status 80000))
 (segment (start 133.604 115.316) (end 134.366 115.316) (width 0.254) (layer B.Cu) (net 2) (status 80000))
 (segment (start 134.366 115.316) (end 134.239 115.41125) (width 0.254) (layer B.Cu) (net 2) (status 80000))
 (segment (start 127.635 99.66325) (end 127.762 99.568) (width 0.254) (layer B.Cu) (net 2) (status 80000))
 (segment (start 127.762 99.568) (end 128.778 98.552) (width 0.254) (layer B.Cu) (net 2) (status 80000))
 (segment (start 128.778 98.552) (end 131.064 98.552) (width 0.254) (layer B.Cu) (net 2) (status 80000))
 (segment (start 131.064 98.552) (end 132.08 99.568) (width 0.254) (layer B.Cu) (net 2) (status 80000))
 (segment (start 132.08 99.568) (end 132.842 99.568) (width 0.254) (layer B.Cu) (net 2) (status 80000))
 (segment (start 132.842 99.568) (end 132.715 99.66325) (width 0.254) (layer B.Cu) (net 2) (status 80000))
 (segment (start 118.364 98.90125) (end 118.364 98.806) (width 0.254) (layer B.Cu) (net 2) (status 80000))
 (segment (start 118.364 98.806) (end 113.792 98.806) (width 0.254) (layer B.Cu) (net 2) (status 80000))
 (segment (start 113.792 98.806) (end 113.665 98.90125) (width 0.254) (layer B.Cu) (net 2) (status 80000))
 (segment (start 123.825 102.45725) (end 123.952 102.362) (width 0.254) (layer F.Cu) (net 20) (status 80000))
 (segment (start 123.952 102.362) (end 120.904 99.314) (width 0.254) (layer F.Cu) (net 20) (status 80000))
 (segment (start 120.904 99.314) (end 120.904 96.36125) (width 0.254) (layer F.Cu) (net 20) (status 80000))
 (segment (start 113.665 109.06125) (end 113.792 108.966) (width 0.254) (layer B.Cu) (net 21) (status 80000))
 (segment (start 113.792 108.966) (end 113.792 109.728) (width 0.254) (layer B.Cu) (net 21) (status 80000))
 (segment (start 113.792 109.728) (end 117.602 113.538) (width 0.254) (layer B.Cu) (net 21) (status 80000))
 (segment (start 117.602 113.538) (end 119.634 113.538) (width 0.254) (layer B.Cu) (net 21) (status 80000))
 (segment (start 119.634 113.538) (end 119.634 113.63325) (width 0.254) (layer B.Cu) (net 21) (status 80000))
 (segment (start 131.191 105.50525) (end 131.318 105.41) (width 0.254) (layer B.Cu) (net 1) (status 80000))
 (segment (start 131.318 105.41) (end 131.318 103.124) (width 0.254) (layer B.Cu) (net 1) (status 80000))
 (segment (start 131.318 103.124) (end 135.382 99.06) (width 0.254) (layer B.Cu) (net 1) (status 80000))
 (segment (start 135.382 99.06) (end 137.16 99.06) (width 0.254) (layer B.Cu) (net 1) (status 80000))
 (segment (start 137.16 99.06) (end 137.033 99.15525) (width 0.254) (layer B.Cu) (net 1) (status 80000))
 (segment (start 153.67 98.90125) (end 153.67 98.806) (width 0.254) (layer B.Cu) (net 18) (status 80000))
 (segment (start 153.67 98.806) (end 152.654 97.79) (width 0.254) (layer B.Cu) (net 18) (status 80000))
 (segment (start 152.654 97.79) (end 148.336 97.79) (width 0.254) (layer B.Cu) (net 18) (status 80000))
 (segment (start 148.336 97.79) (end 148.336 97.88525) (width 0.254) (layer B.Cu) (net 18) (status 80000))
 (segment (start 125.095 99.66325) (end 125.222 99.568) (width 0.254) (layer F.Cu) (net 3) (status 80000))
 (segment (start 125.222 99.568) (end 122.174 96.52) (width 0.254) (layer F.Cu) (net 3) (status 80000))
 (segment (start 122.174 96.52) (end 122.174 95.758) (width 0.254) (layer F.Cu) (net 3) (status 80000))
 (segment (start 122.174 95.758) (end 118.618 92.202) (width 0.254) (layer F.Cu) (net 3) (status 80000))
 (segment (start 118.618 92.202) (end 118.618 89.662) (width 0.254) (layer F.Cu) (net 3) (status 80000))
 (segment (start 118.618 89.662) (end 118.491 89.75725) (width 0.254) (layer F.Cu) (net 3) (status 80000))
 (segment (start 126.111 89.75725) (end 126.238 89.662) (width 0.254) (layer B.Cu) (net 4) (status 80000))
 (segment (start 126.238 89.662) (end 129.032 89.662) (width 0.254) (layer B.Cu) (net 4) (status 80000))
 (segment (start 129.032 89.662) (end 128.905 89.75725) (width 0.254) (layer B.Cu) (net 4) (status 80000))
 (segment (start 125.095 92.04325) (end 125.222 91.948) (width 0.254) (layer F.Cu) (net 9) (status 80000))
 (segment (start 125.222 91.948) (end 125.73 91.948) (width 0.254) (layer F.Cu) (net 9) (status 80000))
 (segment (start 125.73 91.948) (end 126.746 90.932) (width 0.254) (layer F.Cu) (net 9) (status 80000))
 (segment (start 126.746 90.932) (end 132.842 90.932) (width 0.254) (layer F.Cu) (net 9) (status 80000))
 (segment (start 132.842 90.932) (end 134.112 89.662) (width 0.254) (layer F.Cu) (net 9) (status 80000))
 (segment (start 134.112 89.662) (end 133.985 89.75725) (width 0.254) (layer F.Cu) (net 9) (status 80000))
 (segment (start 148.336 110.07725) (end 148.336 109.982) (width 0.254) (layer B.Cu) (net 17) (status 80000))
 (segment (start 148.336 109.982) (end 151.892 106.426) (width 0.254) (layer B.Cu) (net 17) (status 80000))
 (segment (start 151.892 106.426) (end 153.67 106.426) (width 0.254) (layer B.Cu) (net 17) (status 80000))
 (segment (start 153.67 106.426) (end 153.67 106.52125) (width 0.254) (layer B.Cu) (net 17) (status 80000))
 (segment (start 123.825 109.56925) (end 123.952 109.474) (width 0.254) (layer B.Cu) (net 8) (status 80000))
 (segment (start 123.952 109.474) (end 125.73 107.696) (width 0.254) (layer B.Cu) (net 8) (status 80000))
 (segment (start 125.73 107.696) (end 126.746 107.696) (width 0.254) (layer B.Cu) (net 8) (status 80000))
 (segment (start 126.746 107.696) (end 126.619 107.79125) (width 0.254) (layer B.Cu) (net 8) (status 80000))
 (segment (start 134.239 107.79125) (end 134.366 107.696) (width 0.254) (layer B.Cu) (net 15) (status 80000))
 (segment (start 134.366 107.696) (end 136.652 109.982) (width 0.254) (layer B.Cu) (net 15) (status 80000))
 (segment (start 136.652 109.982) (end 143.256 109.982) (width 0.254) (layer B.Cu) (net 15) (status 80000))
 (segment (start 143.256 109.982) (end 143.256 110.07725) (width 0.254) (layer B.Cu) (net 15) (status 80000))
 (segment (start 134.239 107.79125) (end 134.366 107.696) (width 0.254) (layer F.Cu) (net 15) (status 80000))
 (segment (start 134.366 107.696) (end 133.35 106.68) (width 0.254) (layer F.Cu) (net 15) (status 80000))
 (segment (start 133.35 106.68) (end 133.35 103.378) (width 0.254) (layer F.Cu) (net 15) (status 80000))
 (segment (start 133.35 103.378) (end 133.223 103.47325) (width 0.254) (layer F.Cu) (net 15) (status 80000))
 (segment (start 132.715 92.04325) (end 132.842 91.948) (width 0.254) (layer F.Cu) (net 11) (status 80000))
 (segment (start 132.842 91.948) (end 137.16 96.266) (width 0.254) (layer F.Cu) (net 11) (status 80000))
 (segment (start 137.16 96.266) (end 137.16 96.52) (width 0.254) (layer F.Cu) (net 11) (status 80000))
 (segment (start 137.16 96.52) (end 137.033 96.61525) (width 0.254) (layer F.Cu) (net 11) (status 80000))
 (segment (start 137.033 96.61525) (end 137.16 96.52) (width 0.254) (layer B.Cu) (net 11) (status 80000))
 (segment (start 137.16 96.52) (end 138.43 97.79) (width 0.254) (layer B.Cu) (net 11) (status 80000))
 (segment (start 138.43 97.79) (end 143.256 97.79) (width 0.254) (layer B.Cu) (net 11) (status 80000))
 (segment (start 143.256 97.79) (end 143.256 97.88525) (width 0.254) (layer B.Cu) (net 11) (status 80000))
 (segment (start 125.603 118.20525) (end 125.73 118.11) (width 0.254) (layer F.Cu) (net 5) (status 80000))
 (segment (start 125.73 118.11) (end 126.746 117.094) (width 0.254) (layer F.Cu) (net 5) (status 80000))
 (segment (start 126.746 117.094) (end 126.746 115.316) (width 0.254) (layer F.Cu) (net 5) (status 80000))
 (segment (start 126.746 115.316) (end 126.619 115.41125) (width 0.254) (layer F.Cu) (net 5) (status 80000))
 (segment (start 123.825 114.64925) (end 123.952 114.554) (width 0.254) (layer B.Cu) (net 6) (status 80000))
 (segment (start 123.952 114.554) (end 120.396 118.11) (width 0.254) (layer B.Cu) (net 6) (status 80000))
 (segment (start 120.396 118.11) (end 118.11 118.11) (width 0.254) (layer B.Cu) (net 6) (status 80000))
 (segment (start 118.11 118.11) (end 117.983 118.20525) (width 0.254) (layer B.Cu) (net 6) (status 80000))
 (segment (start 128.905 102.45725) (end 129.032 102.362) (width 0.254) (layer F.Cu) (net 10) (status 80000))
 (segment (start 129.032 102.362) (end 130.302 101.092) (width 0.254) (layer F.Cu) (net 10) (status 80000))
 (segment (start 130.302 101.092) (end 130.302 99.568) (width 0.254) (layer F.Cu) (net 10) (status 80000))
 (segment (start 130.302 99.568) (end 130.175 99.66325) (width 0.254) (layer F.Cu) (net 10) (status 80000))
 (segment (start 133.477 118.20525) (end 133.604 118.11) (width 0.254) (layer F.Cu) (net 14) (status 80000))
 (segment (start 133.604 118.11) (end 131.826 116.332) (width 0.254) (layer F.Cu) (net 14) (status 80000))
 (segment (start 131.826 116.332) (end 131.826 115.316) (width 0.254) (layer F.Cu) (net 14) (status 80000))
 (segment (start 131.826 115.316) (end 131.699 115.41125) (width 0.254) (layer F.Cu) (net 14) (status 80000))
 (segment (start 137.541 116.17325) (end 137.668 116.078) (width 0.254) (layer F.Cu) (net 16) (status 80000))
 (segment (start 137.668 116.078) (end 129.286 107.696) (width 0.254) (layer F.Cu) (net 16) (status 80000))
 (segment (start 129.286 107.696) (end 129.159 107.79125) (width 0.254) (layer F.Cu) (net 16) (status 80000))
 (segment (start 138.049 104.23525) (end 138.176 104.14) (width 0.254) (layer B.Cu) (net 7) (status 80000))
 (segment (start 138.176 104.14) (end 137.414 103.378) (width 0.254) (layer B.Cu) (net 7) (status 80000))
 (segment (start 137.414 103.378) (end 135.89 103.378) (width 0.254) (layer B.Cu) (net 7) (status 80000))
 (segment (start 135.89 103.378) (end 135.763 103.47325) (width 0.254) (layer B.Cu) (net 7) (status 80000))
 (segment (start 138.557 90.51925) (end 138.684 90.424) (width 0.254) (layer B.Cu) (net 13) (status 80000))
 (segment (start 138.684 90.424) (end 138.176 90.932) (width 0.254) (layer B.Cu) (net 13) (status 80000))
 (segment (start 138.176 90.932) (end 129.286 90.932) (width 0.254) (layer B.Cu) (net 13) (status 80000))
 (segment (start 129.286 90.932) (end 128.27 91.948) (width 0.254) (layer B.Cu) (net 13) (status 80000))
 (segment (start 128.27 91.948) (end 127.762 91.948) (width 0.254) (layer B.Cu) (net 13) (status 80000))
 (segment (start 127.762 91.948) (end 127.635 92.04325) (width 0.254) (layer B.Cu) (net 13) (status 80000))
 (segment (start 113.665 103.98125) (end 113.792 103.98125) (width 0.254) (layer B.Cu) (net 19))
 (segment (start 118.364 96.36125) (end 118.364 93.82125) (width 0.254) (layer B.Cu) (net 19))
 (segment (start 120.396 98.39325) (end 118.364 96.36125) (width 0.254) (layer B.Cu) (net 19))
 (segment (start 120.396 99.40925) (end 120.396 98.39325) (width 0.254) (layer B.Cu) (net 19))
 (segment (start 119.38 100.42525) (end 120.396 99.40925) (width 0.254) (layer B.Cu) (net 19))
 (segment (start 117.348 100.42525) (end 119.38 100.42525) (width 0.254) (layer B.Cu) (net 19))
 (segment (start 113.792 103.98125) (end 117.348 100.42525) (width 0.254) (layer B.Cu) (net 19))
 (segment (start 128.397 118.20525) (end 128.524 118.11) (width 0.254) (layer B.Cu) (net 22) (status 80000))
 (segment (start 128.524 118.11) (end 127 116.586) (width 0.254) (layer B.Cu) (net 22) (status 80000))
 (segment (start 127 116.586) (end 125.476 116.586) (width 0.254) (layer B.Cu) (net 22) (status 80000))
 (segment (start 125.476 116.586) (end 125.476 114.3) (width 0.254) (layer B.Cu) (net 22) (status 80000))
 (segment (start 125.476 114.3) (end 122.174 110.998) (width 0.254) (layer B.Cu) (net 22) (status 80000))
 (segment (start 122.174 110.998) (end 117.094 110.998) (width 0.254) (layer B.Cu) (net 22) (status 80000))
 (segment (start 117.094 110.998) (end 117.094 111.09325) (width 0.254) (layer B.Cu) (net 22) (status 80000)))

